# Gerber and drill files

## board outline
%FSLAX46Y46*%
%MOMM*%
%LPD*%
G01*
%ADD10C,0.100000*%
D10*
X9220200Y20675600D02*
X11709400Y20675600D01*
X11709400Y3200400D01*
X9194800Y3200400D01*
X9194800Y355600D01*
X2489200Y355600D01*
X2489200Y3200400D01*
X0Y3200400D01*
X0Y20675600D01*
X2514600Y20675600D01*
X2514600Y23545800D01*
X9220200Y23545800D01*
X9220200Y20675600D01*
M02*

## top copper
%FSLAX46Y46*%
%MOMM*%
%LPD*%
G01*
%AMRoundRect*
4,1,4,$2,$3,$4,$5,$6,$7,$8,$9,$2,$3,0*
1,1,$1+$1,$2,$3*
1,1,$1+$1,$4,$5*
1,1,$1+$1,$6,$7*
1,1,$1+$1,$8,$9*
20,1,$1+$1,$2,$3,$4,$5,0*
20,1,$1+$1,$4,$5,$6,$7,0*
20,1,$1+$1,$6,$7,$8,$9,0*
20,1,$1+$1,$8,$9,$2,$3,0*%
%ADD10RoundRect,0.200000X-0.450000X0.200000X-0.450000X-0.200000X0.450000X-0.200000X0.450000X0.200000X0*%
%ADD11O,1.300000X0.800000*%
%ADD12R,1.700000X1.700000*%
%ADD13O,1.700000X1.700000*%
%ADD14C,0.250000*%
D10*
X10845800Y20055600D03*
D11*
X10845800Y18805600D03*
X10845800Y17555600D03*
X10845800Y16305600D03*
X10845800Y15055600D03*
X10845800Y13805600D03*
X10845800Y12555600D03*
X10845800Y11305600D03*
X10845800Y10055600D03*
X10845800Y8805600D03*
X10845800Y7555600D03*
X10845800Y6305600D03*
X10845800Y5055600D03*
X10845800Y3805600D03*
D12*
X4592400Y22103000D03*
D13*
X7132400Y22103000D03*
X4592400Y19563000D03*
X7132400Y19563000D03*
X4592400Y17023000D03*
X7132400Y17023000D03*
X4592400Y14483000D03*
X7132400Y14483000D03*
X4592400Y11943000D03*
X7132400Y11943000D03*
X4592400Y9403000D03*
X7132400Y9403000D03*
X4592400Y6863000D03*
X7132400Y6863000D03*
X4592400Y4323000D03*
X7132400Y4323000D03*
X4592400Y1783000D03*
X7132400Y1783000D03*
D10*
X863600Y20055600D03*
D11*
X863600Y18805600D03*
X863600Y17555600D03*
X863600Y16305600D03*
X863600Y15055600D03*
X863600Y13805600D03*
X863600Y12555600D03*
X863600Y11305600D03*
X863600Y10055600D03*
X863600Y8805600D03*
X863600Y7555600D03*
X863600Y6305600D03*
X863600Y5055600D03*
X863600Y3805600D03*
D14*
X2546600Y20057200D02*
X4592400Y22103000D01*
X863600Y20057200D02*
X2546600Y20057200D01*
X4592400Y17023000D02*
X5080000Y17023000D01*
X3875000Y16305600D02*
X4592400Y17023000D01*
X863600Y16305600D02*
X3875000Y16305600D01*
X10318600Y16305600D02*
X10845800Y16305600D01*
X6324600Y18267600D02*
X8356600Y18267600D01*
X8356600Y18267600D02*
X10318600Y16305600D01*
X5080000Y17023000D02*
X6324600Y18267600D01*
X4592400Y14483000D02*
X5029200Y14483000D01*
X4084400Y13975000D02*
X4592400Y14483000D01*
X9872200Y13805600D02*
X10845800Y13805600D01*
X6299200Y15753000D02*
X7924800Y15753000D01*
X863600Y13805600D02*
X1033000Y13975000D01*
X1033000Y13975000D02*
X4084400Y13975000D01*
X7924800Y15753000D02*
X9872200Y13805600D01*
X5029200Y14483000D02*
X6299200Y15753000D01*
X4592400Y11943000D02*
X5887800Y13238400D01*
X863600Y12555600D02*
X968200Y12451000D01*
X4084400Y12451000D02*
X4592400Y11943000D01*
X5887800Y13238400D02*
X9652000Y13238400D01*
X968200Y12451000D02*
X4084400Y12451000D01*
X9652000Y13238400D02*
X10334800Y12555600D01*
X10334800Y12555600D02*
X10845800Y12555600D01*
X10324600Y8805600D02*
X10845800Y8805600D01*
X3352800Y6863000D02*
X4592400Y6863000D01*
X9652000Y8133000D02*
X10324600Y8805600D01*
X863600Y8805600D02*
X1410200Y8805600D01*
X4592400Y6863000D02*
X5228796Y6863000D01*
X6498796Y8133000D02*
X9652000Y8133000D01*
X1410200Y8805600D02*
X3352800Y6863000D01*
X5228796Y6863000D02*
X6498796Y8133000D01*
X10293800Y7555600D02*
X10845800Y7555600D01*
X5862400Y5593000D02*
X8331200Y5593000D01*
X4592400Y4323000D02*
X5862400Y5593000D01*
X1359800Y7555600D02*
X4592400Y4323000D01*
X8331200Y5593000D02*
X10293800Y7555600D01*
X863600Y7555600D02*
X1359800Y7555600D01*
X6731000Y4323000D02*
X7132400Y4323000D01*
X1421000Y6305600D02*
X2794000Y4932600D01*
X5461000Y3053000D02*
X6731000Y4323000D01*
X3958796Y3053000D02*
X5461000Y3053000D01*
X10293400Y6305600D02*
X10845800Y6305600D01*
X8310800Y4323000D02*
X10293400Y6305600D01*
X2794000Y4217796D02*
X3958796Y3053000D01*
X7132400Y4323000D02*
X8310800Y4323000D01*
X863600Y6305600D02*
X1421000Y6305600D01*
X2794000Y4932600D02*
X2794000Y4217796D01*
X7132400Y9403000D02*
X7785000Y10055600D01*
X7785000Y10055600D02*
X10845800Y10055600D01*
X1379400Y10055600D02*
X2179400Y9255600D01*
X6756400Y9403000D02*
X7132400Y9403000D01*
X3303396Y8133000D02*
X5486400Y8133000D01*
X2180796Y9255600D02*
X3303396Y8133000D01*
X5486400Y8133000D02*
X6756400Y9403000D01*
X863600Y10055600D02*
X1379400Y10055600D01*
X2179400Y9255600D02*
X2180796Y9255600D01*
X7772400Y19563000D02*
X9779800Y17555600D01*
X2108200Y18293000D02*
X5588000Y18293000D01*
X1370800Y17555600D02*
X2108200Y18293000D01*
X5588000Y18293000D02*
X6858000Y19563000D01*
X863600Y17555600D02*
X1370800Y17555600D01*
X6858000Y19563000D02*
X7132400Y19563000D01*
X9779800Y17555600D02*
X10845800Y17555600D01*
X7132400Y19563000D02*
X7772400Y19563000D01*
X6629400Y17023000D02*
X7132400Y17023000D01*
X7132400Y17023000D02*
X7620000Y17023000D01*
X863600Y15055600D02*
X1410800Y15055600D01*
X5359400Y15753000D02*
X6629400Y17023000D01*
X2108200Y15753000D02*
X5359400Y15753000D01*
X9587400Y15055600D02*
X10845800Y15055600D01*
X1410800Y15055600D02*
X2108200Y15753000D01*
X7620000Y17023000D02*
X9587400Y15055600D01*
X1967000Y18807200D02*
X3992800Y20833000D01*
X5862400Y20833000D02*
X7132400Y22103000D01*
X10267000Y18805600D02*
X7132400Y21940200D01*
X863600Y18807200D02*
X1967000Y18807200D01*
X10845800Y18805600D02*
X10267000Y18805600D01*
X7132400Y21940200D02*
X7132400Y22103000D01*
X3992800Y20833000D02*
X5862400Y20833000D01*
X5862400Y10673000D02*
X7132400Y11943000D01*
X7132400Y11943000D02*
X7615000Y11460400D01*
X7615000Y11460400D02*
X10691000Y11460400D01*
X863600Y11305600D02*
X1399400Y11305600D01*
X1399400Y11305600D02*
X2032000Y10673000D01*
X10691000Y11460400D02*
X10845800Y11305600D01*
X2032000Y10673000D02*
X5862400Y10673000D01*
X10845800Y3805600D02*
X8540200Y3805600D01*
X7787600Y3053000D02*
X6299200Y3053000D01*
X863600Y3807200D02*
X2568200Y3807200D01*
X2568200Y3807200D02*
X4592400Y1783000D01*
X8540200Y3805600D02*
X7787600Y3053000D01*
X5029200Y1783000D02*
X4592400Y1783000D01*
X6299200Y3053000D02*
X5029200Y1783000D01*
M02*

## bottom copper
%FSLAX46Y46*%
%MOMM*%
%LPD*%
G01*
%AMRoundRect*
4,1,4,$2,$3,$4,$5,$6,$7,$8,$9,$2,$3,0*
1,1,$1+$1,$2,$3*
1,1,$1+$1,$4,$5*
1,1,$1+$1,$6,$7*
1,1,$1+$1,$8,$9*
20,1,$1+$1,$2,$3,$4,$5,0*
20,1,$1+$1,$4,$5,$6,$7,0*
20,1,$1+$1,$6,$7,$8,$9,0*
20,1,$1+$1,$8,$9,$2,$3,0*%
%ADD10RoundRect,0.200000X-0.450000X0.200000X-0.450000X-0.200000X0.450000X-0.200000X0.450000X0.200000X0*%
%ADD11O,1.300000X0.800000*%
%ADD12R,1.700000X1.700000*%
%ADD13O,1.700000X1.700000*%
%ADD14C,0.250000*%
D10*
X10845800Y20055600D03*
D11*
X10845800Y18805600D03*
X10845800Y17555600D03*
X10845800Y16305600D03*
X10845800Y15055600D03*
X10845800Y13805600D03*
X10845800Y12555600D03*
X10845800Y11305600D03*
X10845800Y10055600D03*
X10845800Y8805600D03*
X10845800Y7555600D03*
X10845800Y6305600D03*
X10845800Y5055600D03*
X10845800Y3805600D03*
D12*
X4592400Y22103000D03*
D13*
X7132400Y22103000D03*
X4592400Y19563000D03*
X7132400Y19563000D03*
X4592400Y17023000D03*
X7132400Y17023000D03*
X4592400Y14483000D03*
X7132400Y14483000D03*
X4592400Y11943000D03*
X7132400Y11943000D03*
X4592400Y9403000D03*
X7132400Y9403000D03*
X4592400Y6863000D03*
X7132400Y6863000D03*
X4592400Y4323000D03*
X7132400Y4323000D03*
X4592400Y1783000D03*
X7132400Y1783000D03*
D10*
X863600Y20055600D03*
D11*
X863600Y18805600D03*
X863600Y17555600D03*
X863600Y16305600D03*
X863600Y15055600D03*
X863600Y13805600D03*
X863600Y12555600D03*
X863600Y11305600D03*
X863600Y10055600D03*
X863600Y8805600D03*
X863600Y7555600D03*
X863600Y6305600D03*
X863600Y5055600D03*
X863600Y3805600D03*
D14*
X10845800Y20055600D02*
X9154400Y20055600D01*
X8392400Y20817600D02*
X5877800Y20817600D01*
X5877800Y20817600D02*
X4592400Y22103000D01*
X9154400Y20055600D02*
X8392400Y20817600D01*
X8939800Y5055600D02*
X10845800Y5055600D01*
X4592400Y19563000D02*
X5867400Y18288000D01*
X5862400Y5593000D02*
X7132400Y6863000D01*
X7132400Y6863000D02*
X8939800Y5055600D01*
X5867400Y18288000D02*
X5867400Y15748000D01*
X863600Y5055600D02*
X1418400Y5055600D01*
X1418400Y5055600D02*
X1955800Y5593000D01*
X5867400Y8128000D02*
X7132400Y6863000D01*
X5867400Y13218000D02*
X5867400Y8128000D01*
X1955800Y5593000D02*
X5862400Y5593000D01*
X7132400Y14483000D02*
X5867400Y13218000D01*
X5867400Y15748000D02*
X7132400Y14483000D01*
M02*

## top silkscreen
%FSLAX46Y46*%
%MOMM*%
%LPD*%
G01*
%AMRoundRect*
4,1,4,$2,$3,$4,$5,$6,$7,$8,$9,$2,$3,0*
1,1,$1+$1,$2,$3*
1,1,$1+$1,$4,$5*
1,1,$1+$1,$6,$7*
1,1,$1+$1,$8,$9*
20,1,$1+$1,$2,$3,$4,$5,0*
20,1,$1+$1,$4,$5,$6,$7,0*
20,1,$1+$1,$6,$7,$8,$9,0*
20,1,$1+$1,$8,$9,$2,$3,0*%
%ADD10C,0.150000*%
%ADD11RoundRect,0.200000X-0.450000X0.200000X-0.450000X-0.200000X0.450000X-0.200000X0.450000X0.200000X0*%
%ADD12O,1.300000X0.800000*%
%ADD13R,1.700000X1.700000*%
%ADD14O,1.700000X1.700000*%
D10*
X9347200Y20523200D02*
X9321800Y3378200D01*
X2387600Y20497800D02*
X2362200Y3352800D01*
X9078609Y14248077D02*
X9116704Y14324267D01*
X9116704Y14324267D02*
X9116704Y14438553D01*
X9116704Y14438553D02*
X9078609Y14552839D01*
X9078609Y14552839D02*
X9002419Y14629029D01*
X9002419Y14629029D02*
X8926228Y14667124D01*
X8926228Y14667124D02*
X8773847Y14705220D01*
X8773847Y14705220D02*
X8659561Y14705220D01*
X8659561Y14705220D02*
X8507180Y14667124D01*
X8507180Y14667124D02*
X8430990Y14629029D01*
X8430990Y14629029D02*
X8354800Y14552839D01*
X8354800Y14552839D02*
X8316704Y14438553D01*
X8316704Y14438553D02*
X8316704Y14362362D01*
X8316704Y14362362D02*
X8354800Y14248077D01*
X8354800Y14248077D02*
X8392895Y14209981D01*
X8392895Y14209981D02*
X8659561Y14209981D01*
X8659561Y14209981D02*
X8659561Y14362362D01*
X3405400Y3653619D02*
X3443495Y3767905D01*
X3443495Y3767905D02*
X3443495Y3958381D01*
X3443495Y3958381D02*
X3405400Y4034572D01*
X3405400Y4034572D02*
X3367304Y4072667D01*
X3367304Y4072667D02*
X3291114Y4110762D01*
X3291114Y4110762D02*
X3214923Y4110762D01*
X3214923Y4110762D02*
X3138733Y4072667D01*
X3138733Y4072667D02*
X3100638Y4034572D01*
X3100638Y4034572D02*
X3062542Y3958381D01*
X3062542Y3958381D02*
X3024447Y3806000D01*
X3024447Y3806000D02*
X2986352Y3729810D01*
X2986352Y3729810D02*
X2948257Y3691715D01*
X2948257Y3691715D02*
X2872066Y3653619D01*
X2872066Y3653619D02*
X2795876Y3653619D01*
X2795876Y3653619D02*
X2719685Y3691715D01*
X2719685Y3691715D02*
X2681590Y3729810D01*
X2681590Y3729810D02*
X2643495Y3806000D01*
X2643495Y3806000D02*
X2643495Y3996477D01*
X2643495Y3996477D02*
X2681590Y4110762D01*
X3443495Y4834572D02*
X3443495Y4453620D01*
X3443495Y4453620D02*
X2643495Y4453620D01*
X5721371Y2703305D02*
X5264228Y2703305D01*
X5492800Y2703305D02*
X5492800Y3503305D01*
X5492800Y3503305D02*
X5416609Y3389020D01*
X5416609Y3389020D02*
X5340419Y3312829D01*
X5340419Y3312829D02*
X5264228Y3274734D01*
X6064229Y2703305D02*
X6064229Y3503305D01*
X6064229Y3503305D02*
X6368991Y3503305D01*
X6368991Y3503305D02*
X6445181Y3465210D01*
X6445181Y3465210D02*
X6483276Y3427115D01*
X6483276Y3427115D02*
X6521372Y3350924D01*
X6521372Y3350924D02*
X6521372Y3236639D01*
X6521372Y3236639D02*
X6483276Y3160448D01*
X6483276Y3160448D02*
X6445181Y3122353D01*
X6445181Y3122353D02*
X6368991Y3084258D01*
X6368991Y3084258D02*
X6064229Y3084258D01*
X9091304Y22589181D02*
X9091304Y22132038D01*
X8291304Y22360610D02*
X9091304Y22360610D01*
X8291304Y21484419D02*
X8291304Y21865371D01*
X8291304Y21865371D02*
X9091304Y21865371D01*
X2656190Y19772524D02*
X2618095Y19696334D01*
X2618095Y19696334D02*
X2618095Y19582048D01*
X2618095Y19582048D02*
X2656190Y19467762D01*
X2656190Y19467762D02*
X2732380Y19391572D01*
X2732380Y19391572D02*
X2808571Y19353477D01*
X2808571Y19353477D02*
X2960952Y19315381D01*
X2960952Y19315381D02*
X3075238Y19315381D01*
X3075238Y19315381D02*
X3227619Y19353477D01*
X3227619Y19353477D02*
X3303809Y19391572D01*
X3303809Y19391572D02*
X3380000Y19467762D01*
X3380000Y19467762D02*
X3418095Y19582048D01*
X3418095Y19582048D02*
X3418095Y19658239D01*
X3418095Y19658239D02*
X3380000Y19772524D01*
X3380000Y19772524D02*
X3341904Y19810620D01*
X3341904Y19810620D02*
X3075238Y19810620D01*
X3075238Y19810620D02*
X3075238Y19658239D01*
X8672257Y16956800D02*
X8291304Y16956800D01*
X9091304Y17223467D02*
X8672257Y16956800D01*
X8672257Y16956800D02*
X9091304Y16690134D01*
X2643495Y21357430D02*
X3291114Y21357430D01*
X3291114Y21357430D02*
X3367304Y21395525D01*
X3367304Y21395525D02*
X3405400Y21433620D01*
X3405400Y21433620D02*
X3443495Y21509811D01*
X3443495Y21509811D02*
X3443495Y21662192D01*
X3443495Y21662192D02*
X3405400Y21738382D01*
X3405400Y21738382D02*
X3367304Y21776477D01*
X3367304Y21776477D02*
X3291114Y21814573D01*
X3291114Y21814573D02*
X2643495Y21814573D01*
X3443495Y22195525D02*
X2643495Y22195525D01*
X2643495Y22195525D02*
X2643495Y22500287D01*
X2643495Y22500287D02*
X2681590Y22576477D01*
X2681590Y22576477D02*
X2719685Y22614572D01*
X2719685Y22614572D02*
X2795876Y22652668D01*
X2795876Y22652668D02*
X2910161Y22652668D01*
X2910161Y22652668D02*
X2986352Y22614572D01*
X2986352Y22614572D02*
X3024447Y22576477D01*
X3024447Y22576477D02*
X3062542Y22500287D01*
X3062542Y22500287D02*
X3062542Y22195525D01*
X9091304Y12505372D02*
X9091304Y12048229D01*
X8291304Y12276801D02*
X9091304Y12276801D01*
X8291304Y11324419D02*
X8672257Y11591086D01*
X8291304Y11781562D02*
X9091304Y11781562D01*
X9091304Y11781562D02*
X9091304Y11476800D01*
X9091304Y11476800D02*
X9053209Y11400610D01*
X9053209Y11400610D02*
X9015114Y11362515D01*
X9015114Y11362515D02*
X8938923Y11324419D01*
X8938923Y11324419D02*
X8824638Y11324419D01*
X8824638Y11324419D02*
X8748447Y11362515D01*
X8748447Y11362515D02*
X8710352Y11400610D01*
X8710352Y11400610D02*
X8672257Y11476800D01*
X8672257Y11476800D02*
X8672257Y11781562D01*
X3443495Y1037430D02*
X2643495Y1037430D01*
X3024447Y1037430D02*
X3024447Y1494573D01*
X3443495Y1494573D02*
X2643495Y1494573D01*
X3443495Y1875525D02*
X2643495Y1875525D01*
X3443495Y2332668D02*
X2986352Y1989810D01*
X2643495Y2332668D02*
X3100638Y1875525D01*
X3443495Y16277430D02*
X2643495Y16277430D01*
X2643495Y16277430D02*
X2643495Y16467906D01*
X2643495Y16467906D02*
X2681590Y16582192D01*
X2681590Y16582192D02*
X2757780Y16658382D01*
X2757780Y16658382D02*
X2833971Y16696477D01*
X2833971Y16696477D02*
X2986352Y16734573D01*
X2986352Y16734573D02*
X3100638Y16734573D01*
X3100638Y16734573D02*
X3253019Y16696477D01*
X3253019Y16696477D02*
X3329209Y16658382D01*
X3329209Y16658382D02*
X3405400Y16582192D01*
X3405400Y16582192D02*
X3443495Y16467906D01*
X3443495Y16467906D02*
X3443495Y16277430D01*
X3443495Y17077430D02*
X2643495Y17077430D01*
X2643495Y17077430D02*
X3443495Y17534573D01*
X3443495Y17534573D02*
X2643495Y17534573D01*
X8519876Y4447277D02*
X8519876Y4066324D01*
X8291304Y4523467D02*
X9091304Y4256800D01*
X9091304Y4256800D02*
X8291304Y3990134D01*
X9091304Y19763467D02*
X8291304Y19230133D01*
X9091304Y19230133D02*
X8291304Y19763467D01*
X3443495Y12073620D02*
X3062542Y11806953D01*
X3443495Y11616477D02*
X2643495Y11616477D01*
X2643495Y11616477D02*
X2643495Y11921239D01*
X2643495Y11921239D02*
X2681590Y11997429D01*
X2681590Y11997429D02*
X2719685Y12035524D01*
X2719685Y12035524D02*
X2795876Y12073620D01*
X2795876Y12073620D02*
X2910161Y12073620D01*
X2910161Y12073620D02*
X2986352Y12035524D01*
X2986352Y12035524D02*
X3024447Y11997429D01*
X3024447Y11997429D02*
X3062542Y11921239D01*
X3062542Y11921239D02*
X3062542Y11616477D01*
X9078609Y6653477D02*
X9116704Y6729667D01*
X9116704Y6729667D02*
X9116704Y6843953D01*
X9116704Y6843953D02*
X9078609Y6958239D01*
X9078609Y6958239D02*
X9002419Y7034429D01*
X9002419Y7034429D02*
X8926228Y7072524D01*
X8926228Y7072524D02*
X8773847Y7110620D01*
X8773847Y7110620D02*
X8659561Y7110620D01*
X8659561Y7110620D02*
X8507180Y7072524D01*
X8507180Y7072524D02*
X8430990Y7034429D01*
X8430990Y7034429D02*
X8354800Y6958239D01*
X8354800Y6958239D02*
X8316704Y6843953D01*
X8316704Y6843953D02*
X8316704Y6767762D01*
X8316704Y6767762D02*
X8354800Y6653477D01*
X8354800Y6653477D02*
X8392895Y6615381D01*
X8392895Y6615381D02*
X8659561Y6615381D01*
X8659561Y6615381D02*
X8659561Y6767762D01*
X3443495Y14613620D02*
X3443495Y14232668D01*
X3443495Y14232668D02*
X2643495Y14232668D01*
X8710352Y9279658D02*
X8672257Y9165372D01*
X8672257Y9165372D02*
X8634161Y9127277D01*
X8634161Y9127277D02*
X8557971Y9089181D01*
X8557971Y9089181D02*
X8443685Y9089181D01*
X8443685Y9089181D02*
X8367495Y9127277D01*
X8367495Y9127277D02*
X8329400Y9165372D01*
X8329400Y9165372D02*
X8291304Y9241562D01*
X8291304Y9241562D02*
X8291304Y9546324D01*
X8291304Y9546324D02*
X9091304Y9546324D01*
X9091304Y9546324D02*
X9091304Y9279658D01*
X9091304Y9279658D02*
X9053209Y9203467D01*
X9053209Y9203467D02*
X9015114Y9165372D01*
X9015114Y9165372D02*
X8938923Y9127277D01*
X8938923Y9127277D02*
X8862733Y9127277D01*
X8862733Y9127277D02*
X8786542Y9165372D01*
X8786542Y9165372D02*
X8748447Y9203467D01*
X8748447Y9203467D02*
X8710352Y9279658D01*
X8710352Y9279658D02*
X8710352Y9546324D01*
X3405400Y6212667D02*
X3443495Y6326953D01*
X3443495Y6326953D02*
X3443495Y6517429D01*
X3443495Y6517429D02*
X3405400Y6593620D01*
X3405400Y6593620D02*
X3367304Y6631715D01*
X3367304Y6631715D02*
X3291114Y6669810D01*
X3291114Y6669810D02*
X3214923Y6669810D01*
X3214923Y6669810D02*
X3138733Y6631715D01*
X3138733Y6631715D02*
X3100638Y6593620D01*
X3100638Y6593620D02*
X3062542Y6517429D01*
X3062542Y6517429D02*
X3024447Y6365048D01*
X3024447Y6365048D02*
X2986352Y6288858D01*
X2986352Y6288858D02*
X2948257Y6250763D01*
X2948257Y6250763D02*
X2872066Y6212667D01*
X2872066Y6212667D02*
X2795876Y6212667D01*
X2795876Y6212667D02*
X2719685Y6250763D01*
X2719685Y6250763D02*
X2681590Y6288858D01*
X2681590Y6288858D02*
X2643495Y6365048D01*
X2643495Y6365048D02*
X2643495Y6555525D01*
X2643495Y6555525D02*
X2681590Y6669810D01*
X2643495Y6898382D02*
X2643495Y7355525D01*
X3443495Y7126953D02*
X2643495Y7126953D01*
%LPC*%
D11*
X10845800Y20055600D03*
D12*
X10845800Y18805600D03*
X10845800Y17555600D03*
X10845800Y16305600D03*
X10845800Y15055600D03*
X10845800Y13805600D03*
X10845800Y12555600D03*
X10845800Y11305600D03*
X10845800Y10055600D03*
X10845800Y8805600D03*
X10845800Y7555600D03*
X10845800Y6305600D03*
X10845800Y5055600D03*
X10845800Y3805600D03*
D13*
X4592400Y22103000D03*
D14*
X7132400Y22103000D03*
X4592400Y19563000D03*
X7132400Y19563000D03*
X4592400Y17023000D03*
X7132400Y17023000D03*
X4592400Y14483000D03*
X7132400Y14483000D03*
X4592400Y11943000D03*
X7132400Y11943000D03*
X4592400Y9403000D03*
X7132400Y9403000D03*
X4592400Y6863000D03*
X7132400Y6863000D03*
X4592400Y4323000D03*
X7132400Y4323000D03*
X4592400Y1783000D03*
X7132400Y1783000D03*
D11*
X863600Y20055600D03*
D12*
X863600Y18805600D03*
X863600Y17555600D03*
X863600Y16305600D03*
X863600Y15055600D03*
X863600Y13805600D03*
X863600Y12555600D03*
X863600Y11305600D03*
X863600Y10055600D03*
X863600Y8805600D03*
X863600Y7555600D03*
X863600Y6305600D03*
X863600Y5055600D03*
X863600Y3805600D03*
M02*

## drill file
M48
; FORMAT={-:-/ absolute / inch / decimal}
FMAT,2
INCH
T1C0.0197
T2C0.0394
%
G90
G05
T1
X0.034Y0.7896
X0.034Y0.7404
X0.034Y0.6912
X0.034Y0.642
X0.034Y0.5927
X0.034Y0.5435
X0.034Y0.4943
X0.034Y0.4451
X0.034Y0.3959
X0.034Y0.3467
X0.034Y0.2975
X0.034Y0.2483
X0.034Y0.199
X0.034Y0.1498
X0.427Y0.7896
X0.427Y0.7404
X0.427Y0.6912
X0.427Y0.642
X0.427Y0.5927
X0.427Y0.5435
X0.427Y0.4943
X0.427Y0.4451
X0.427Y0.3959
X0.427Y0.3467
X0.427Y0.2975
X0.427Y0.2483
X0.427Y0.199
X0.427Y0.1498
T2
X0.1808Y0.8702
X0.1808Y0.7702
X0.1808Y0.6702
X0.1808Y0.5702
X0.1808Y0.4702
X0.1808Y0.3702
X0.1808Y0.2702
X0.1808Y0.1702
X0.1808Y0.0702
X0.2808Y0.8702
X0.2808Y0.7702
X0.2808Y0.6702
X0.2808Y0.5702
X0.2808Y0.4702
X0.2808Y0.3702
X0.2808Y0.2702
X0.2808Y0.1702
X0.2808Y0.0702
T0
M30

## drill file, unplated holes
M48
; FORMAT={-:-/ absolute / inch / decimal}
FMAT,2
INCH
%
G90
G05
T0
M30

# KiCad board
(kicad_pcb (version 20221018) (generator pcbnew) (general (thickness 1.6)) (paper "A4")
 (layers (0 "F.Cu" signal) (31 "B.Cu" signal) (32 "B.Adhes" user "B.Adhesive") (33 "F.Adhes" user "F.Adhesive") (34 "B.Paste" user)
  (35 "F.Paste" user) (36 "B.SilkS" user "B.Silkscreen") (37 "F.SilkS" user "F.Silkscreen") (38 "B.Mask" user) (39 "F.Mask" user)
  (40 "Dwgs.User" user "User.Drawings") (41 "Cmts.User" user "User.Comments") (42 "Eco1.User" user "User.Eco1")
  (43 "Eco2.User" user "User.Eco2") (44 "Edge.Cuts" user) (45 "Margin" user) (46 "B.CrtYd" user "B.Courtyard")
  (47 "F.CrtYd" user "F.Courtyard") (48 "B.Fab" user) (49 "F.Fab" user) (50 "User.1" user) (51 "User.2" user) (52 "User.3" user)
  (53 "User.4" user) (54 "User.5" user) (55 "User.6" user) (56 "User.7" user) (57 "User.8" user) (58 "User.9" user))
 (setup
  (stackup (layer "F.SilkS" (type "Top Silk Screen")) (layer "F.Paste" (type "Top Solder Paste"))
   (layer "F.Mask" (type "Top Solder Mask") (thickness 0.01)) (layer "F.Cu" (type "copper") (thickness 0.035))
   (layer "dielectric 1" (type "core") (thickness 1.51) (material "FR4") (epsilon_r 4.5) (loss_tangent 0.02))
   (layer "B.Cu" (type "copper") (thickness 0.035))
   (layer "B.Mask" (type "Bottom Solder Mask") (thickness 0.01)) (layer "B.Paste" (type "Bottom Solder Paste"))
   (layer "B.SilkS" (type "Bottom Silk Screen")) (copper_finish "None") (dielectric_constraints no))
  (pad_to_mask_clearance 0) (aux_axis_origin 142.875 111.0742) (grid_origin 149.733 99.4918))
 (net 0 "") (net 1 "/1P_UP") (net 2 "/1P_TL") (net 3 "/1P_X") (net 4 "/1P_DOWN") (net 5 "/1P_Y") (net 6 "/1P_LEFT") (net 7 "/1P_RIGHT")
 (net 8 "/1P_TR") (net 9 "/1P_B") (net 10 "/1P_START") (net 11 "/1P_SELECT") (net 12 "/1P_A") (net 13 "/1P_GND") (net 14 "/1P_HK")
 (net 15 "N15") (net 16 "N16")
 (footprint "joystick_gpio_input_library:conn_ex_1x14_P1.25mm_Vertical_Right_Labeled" (layer "B.Cu") (at 153.7208 91.0186 -90)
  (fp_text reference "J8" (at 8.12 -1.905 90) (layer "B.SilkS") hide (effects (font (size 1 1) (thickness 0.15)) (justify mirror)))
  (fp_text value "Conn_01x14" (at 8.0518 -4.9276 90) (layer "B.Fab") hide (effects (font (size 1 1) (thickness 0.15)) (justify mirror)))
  (pad "1" thru_hole roundrect (at 0 0 270) (size 0.8 1.3) (drill 0.5) (layers "*.Cu" "*.Mask") (roundrect_rratio 0.25) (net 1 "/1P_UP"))
  (pad "2" thru_hole oval (at 1.25 0 270) (size 0.8 1.3) (drill 0.5) (layers "*.Cu" "*.Mask") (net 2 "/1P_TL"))
  (pad "3" thru_hole oval (at 2.5 0 270) (size 0.8 1.3) (drill 0.5) (layers "*.Cu" "*.Mask") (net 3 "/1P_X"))
  (pad "4" thru_hole oval (at 3.75 0 270) (size 0.8 1.3) (drill 0.5) (layers "*.Cu" "*.Mask") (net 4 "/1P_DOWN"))
  (pad "5" thru_hole oval (at 5 0 270) (size 0.8 1.3) (drill 0.5) (layers "*.Cu" "*.Mask") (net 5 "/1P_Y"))
  (pad "6" thru_hole oval (at 6.25 0 270) (size 0.8 1.3) (drill 0.5) (layers "*.Cu" "*.Mask") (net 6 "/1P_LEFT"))
  (pad "7" thru_hole oval (at 7.5 0 270) (size 0.8 1.3) (drill 0.5) (layers "*.Cu" "*.Mask") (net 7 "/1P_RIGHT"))
  (pad "8" thru_hole oval (at 8.75 0 270) (size 0.8 1.3) (drill 0.5) (layers "*.Cu" "*.Mask") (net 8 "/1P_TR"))
  (pad "9" thru_hole oval (at 10 0 270) (size 0.8 1.3) (drill 0.5) (layers "*.Cu" "*.Mask") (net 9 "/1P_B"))
  (pad "10" thru_hole oval (at 11.25 0 270) (size 0.8 1.3) (drill 0.5) (layers "*.Cu" "*.Mask") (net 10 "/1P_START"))
  (pad "11" thru_hole oval (at 12.5 0 270) (size 0.8 1.3) (drill 0.5) (layers "*.Cu" "*.Mask") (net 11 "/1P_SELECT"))
  (pad "12" thru_hole oval (at 13.75 0 270) (size 0.8 1.3) (drill 0.5) (layers "*.Cu" "*.Mask") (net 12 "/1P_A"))
  (pad "13" thru_hole oval (at 15 0 270) (size 0.8 1.3) (drill 0.5) (layers "*.Cu" "*.Mask") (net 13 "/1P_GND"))
  (pad "14" thru_hole oval (at 16.25 0 270) (size 0.8 1.3) (drill 0.5) (layers "*.Cu" "*.Mask") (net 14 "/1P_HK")))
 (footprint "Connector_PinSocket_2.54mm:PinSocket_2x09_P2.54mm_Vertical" (layer "B.Cu") (at 147.4674 88.9712 180)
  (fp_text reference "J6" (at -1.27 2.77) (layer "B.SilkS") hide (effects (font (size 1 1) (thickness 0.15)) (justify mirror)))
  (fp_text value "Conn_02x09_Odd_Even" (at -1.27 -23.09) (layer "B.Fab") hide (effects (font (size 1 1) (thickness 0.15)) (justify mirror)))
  (pad "1" thru_hole rect (at 0 0 180) (size 1.7 1.7) (drill 1) (layers "*.Cu" "*.Mask") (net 1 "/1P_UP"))
  (pad "2" thru_hole oval (at -2.54 0 180) (size 1.7 1.7) (drill 1) (layers "*.Cu" "*.Mask") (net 2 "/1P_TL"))
  (pad "3" thru_hole oval (at 0 -2.54 180) (size 1.7 1.7) (drill 1) (layers "*.Cu" "*.Mask") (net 13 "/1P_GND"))
  (pad "4" thru_hole oval (at -2.54 -2.54 180) (size 1.7 1.7) (drill 1) (layers "*.Cu" "*.Mask") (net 3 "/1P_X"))
  (pad "5" thru_hole oval (at 0 -5.08 180) (size 1.7 1.7) (drill 1) (layers "*.Cu" "*.Mask") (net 4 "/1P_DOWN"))
  (pad "6" thru_hole oval (at -2.54 -5.08 180) (size 1.7 1.7) (drill 1) (layers "*.Cu" "*.Mask") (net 5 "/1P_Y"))
  (pad "7" thru_hole oval (at 0 -7.62 180) (size 1.7 1.7) (drill 1) (layers "*.Cu" "*.Mask") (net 6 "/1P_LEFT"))
  (pad "8" thru_hole oval (at -2.54 -7.62 180) (size 1.7 1.7) (drill 1) (layers "*.Cu" "*.Mask") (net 13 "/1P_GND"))
  (pad "9" thru_hole oval (at 0 -10.16 180) (size 1.7 1.7) (drill 1) (layers "*.Cu" "*.Mask") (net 7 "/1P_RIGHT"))
  (pad "10" thru_hole oval (at -2.54 -10.16 180) (size 1.7 1.7) (drill 1) (layers "*.Cu" "*.Mask") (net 8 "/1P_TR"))
  (pad "11" thru_hole oval (at 0 -12.7 180) (size 1.7 1.7) (drill 1) (layers "*.Cu" "*.Mask") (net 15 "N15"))
  (pad "12" thru_hole oval (at -2.54 -12.7 180) (size 1.7 1.7) (drill 1) (layers "*.Cu" "*.Mask") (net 9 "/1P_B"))
  (pad "13" thru_hole oval (at 0 -15.24 180) (size 1.7 1.7) (drill 1) (layers "*.Cu" "*.Mask") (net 10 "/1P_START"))
  (pad "14" thru_hole oval (at -2.54 -15.24 180) (size 1.7 1.7) (drill 1) (layers "*.Cu" "*.Mask") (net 13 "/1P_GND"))
  (pad "15" thru_hole oval (at 0 -17.78 180) (size 1.7 1.7) (drill 1) (layers "*.Cu" "*.Mask") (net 11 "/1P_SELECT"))
  (pad "16" thru_hole oval (at -2.54 -17.78 180) (size 1.7 1.7) (drill 1) (layers "*.Cu" "*.Mask") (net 12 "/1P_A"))
  (pad "17" thru_hole oval (at 0 -20.32 180) (size 1.7 1.7) (drill 1) (layers "*.Cu" "*.Mask") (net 14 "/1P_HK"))
  (pad "18" thru_hole oval (at -2.54 -20.32 180) (size 1.7 1.7) (drill 1) (layers "*.Cu" "*.Mask") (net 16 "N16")))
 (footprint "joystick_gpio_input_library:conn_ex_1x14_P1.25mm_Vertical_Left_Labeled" (layer "B.Cu") (at 143.7386 91.0186 -90)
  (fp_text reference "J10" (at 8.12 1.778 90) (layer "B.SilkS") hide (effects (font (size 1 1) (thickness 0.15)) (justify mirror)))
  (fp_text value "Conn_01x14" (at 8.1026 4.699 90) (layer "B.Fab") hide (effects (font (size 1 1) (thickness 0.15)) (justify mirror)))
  (pad "1" thru_hole roundrect (at 0 0 270) (size 0.8 1.3) (drill 0.5) (layers "*.Cu" "*.Mask") (roundrect_rratio 0.25) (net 1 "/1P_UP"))
  (pad "2" thru_hole oval (at 1.25 0 270) (size 0.8 1.3) (drill 0.5) (layers "*.Cu" "*.Mask") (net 2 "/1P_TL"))
  (pad "3" thru_hole oval (at 2.5 0 270) (size 0.8 1.3) (drill 0.5) (layers "*.Cu" "*.Mask") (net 3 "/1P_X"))
  (pad "4" thru_hole oval (at 3.75 0 270) (size 0.8 1.3) (drill 0.5) (layers "*.Cu" "*.Mask") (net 4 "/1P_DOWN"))
  (pad "5" thru_hole oval (at 5 0 270) (size 0.8 1.3) (drill 0.5) (layers "*.Cu" "*.Mask") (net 5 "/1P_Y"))
  (pad "6" thru_hole oval (at 6.25 0 270) (size 0.8 1.3) (drill 0.5) (layers "*.Cu" "*.Mask") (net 6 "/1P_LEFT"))
  (pad "7" thru_hole oval (at 7.5 0 270) (size 0.8 1.3) (drill 0.5) (layers "*.Cu" "*.Mask") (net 7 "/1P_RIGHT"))
  (pad "8" thru_hole oval (at 8.75 0 270) (size 0.8 1.3) (drill 0.5) (layers "*.Cu" "*.Mask") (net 8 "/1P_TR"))
  (pad "9" thru_hole oval (at 10 0 270) (size 0.8 1.3) (drill 0.5) (layers "*.Cu" "*.Mask") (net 9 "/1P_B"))
  (pad "10" thru_hole oval (at 11.25 0 270) (size 0.8 1.3) (drill 0.5) (layers "*.Cu" "*.Mask") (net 10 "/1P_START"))
  (pad "11" thru_hole oval (at 12.5 0 270) (size 0.8 1.3) (drill 0.5) (layers "*.Cu" "*.Mask") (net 11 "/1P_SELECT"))
  (pad "12" thru_hole oval (at 13.75 0 270) (size 0.8 1.3) (drill 0.5) (layers "*.Cu" "*.Mask") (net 12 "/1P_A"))
  (pad "13" thru_hole oval (at 15 0 270) (size 0.8 1.3) (drill 0.5) (layers "*.Cu" "*.Mask") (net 13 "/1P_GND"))
  (pad "14" thru_hole oval (at 16.25 0 270) (size 0.8 1.3) (drill 0.5) (layers "*.Cu" "*.Mask") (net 14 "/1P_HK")))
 (gr_line (start 152.2222 90.551) (end 152.1968 107.696) (stroke (width 0.15) (type default)) (layer "F.SilkS"))
 (gr_line (start 145.2626 90.5764) (end 145.2372 107.7214) (stroke (width 0.15) (type default)) (layer "F.SilkS"))
 (gr_poly
  (pts (xy 152.0952 87.5284) (xy 145.3896 87.5284) (xy 145.3896 90.3986) (xy 142.875 90.3986) (xy 142.875 107.8738) (xy 145.3642 107.8738)
   (xy 145.3642 110.7186) (xy 152.0698 110.7186) (xy 152.0698 107.8738) (xy 154.5844 107.8738) (xy 154.5844 90.3986) (xy 152.0952 90.3986))
  (stroke (width 0.1) (type solid)) (fill none) (layer "Edge.Cuts"))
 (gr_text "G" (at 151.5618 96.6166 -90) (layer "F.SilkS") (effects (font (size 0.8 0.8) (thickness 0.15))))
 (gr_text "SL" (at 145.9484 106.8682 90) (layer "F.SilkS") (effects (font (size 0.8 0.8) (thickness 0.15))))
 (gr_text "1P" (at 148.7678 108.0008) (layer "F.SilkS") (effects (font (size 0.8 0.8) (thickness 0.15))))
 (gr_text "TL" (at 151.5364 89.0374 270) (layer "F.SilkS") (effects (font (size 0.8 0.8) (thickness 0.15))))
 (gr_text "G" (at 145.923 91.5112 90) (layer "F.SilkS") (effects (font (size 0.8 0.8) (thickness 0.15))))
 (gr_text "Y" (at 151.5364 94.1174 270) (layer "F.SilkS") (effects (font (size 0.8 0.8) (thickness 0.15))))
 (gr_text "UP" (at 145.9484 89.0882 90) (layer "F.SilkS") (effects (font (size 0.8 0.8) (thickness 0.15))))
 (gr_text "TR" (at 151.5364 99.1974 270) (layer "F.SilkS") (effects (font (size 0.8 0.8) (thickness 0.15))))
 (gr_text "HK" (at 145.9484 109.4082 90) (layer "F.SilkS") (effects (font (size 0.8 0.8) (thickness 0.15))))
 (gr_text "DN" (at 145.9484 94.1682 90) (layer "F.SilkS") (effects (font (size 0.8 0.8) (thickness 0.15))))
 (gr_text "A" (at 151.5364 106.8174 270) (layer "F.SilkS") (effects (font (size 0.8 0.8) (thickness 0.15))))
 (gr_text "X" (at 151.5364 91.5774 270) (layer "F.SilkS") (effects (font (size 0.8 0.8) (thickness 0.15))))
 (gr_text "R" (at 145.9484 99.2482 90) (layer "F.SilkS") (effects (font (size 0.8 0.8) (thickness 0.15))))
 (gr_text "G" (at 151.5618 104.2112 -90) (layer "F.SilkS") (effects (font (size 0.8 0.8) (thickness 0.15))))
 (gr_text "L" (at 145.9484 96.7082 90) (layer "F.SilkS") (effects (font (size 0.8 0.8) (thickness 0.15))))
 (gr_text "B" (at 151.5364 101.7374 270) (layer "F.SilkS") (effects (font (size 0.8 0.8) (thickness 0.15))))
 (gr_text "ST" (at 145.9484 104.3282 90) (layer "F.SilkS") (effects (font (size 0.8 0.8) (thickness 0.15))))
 (segment (start 145.4216 91.017) (end 147.4674 88.9712) (width 0.25) (layer "F.Cu") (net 1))
 (segment (start 143.7386 91.017) (end 145.4216 91.017) (width 0.25) (layer "F.Cu") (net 1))
 (segment (start 153.7208 91.0186) (end 152.0294 91.0186) (width 0.25) (layer "B.Cu") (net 1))
 (segment (start 151.2674 90.2566) (end 148.7528 90.2566) (width 0.25) (layer "B.Cu") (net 1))
 (segment (start 148.7528 90.2566) (end 147.4674 88.9712) (width 0.25) (layer "B.Cu") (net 1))
 (segment (start 152.0294 91.0186) (end 151.2674 90.2566) (width 0.25) (layer "B.Cu") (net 1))
 (segment (start 147.4674 94.0512) (end 147.955 94.0512) (width 0.25) (layer "F.Cu") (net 4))
 (segment (start 146.75 94.7686) (end 147.4674 94.0512) (width 0.25) (layer "F.Cu") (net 4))
 (segment (start 143.7386 94.7686) (end 146.75 94.7686) (width 0.25) (layer "F.Cu") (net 4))
 (segment (start 153.1936 94.7686) (end 153.7208 94.7686) (width 0.25) (layer "F.Cu") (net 4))
 (segment (start 149.1996 92.8066) (end 151.2316 92.8066) (width 0.25) (layer "F.Cu") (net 4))
 (segment (start 151.2316 92.8066) (end 153.1936 94.7686) (width 0.25) (layer "F.Cu") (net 4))
 (segment (start 147.955 94.0512) (end 149.1996 92.8066) (width 0.25) (layer "F.Cu") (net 4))
 (segment (start 147.4674 96.5912) (end 147.9042 96.5912) (width 0.25) (layer "F.Cu") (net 6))
 (segment (start 146.9594 97.0992) (end 147.4674 96.5912) (width 0.25) (layer "F.Cu") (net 6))
 (segment (start 152.7472 97.2686) (end 153.7208 97.2686) (width 0.25) (layer "F.Cu") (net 6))
 (segment (start 149.1742 95.3212) (end 150.7998 95.3212) (width 0.25) (layer "F.Cu") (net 6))
 (segment (start 143.7386 97.2686) (end 143.908 97.0992) (width 0.25) (layer "F.Cu") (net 6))
 (segment (start 143.908 97.0992) (end 146.9594 97.0992) (width 0.25) (layer "F.Cu") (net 6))
 (segment (start 150.7998 95.3212) (end 152.7472 97.2686) (width 0.25) (layer "F.Cu") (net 6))
 (segment (start 147.9042 96.5912) (end 149.1742 95.3212) (width 0.25) (layer "F.Cu") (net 6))
 (segment (start 147.4674 99.1312) (end 148.7628 97.8358) (width 0.25) (layer "F.Cu") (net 7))
 (segment (start 143.7386 98.5186) (end 143.8432 98.6232) (width 0.25) (layer "F.Cu") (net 7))
 (segment (start 146.9594 98.6232) (end 147.4674 99.1312) (width 0.25) (layer "F.Cu") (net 7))
 (segment (start 148.7628 97.8358) (end 152.527 97.8358) (width 0.25) (layer "F.Cu") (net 7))
 (segment (start 143.8432 98.6232) (end 146.9594 98.6232) (width 0.25) (layer "F.Cu") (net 7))
 (segment (start 152.527 97.8358) (end 153.2098 98.5186) (width 0.25) (layer "F.Cu") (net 7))
 (segment (start 153.2098 98.5186) (end 153.7208 98.5186) (width 0.25) (layer "F.Cu") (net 7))
 (segment (start 153.1996 102.2686) (end 153.7208 102.2686) (width 0.25) (layer "F.Cu") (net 10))
 (segment (start 146.2278 104.2112) (end 147.4674 104.2112) (width 0.25) (layer "F.Cu") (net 10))
 (segment (start 152.527 102.9412) (end 153.1996 102.2686) (width 0.25) (layer "F.Cu") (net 10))
 (segment (start 143.7386 102.2686) (end 144.2852 102.2686) (width 0.25) (layer "F.Cu") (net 10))
 (segment (start 147.4674 104.2112) (end 148.103796 104.2112) (width 0.25) (layer "F.Cu") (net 10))
 (segment (start 149.373796 102.9412) (end 152.527 102.9412) (width 0.25) (layer "F.Cu") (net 10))
 (segment (start 144.2852 102.2686) (end 146.2278 104.2112) (width 0.25) (layer "F.Cu") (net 10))
 (segment (start 148.103796 104.2112) (end 149.373796 102.9412) (width 0.25) (layer "F.Cu") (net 10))
 (segment (start 153.1688 103.5186) (end 153.7208 103.5186) (width 0.25) (layer "F.Cu") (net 11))
 (segment (start 148.7374 105.4812) (end 151.2062 105.4812) (width 0.25) (layer "F.Cu") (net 11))
 (segment (start 147.4674 106.7512) (end 148.7374 105.4812) (width 0.25) (layer "F.Cu") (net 11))
 (segment (start 144.2348 103.5186) (end 147.4674 106.7512) (width 0.25) (layer "F.Cu") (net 11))
 (segment (start 151.2062 105.4812) (end 153.1688 103.5186) (width 0.25) (layer "F.Cu") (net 11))
 (segment (start 143.7386 103.5186) (end 144.2348 103.5186) (width 0.25) (layer "F.Cu") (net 11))
 (segment (start 149.606 106.7512) (end 150.0074 106.7512) (width 0.25) (layer "F.Cu") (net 12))
 (segment (start 144.296 104.7686) (end 145.669 106.1416) (width 0.25) (layer "F.Cu") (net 12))
 (segment (start 148.336 108.0212) (end 149.606 106.7512) (width 0.25) (layer "F.Cu") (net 12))
 (segment (start 146.833796 108.0212) (end 148.336 108.0212) (width 0.25) (layer "F.Cu") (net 12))
 (segment (start 153.1684 104.7686) (end 153.7208 104.7686) (width 0.25) (layer "F.Cu") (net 12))
 (segment (start 151.1858 106.7512) (end 153.1684 104.7686) (width 0.25) (layer "F.Cu") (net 12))
 (segment (start 145.669 106.856404) (end 146.833796 108.0212) (width 0.25) (layer "F.Cu") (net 12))
 (segment (start 150.0074 106.7512) (end 151.1858 106.7512) (width 0.25) (layer "F.Cu") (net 12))
 (segment (start 143.7386 104.7686) (end 144.296 104.7686) (width 0.25) (layer "F.Cu") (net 12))
 (segment (start 145.669 106.1416) (end 145.669 106.856404) (width 0.25) (layer "F.Cu") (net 12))
 (segment (start 150.0074 101.6712) (end 150.66 101.0186) (width 0.25) (layer "F.Cu") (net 9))
 (segment (start 150.66 101.0186) (end 153.7208 101.0186) (width 0.25) (layer "F.Cu") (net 9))
 (segment (start 144.2544 101.0186) (end 145.0544 101.8186) (width 0.25) (layer "F.Cu") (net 9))
 (segment (start 149.6314 101.6712) (end 150.0074 101.6712) (width 0.25) (layer "F.Cu") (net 9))
 (segment (start 146.178396 102.9412) (end 148.3614 102.9412) (width 0.25) (layer "F.Cu") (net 9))
 (segment (start 145.055796 101.8186) (end 146.178396 102.9412) (width 0.25) (layer "F.Cu") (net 9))
 (segment (start 148.3614 102.9412) (end 149.6314 101.6712) (width 0.25) (layer "F.Cu") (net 9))
 (segment (start 143.7386 101.0186) (end 144.2544 101.0186) (width 0.25) (layer "F.Cu") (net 9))
 (segment (start 145.0544 101.8186) (end 145.055796 101.8186) (width 0.25) (layer "F.Cu") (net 9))
 (segment (start 150.6474 91.5112) (end 152.6548 93.5186) (width 0.25) (layer "F.Cu") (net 3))
 (segment (start 144.9832 92.7812) (end 148.463 92.7812) (width 0.25) (layer "F.Cu") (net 3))
 (segment (start 144.2458 93.5186) (end 144.9832 92.7812) (width 0.25) (layer "F.Cu") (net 3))
 (segment (start 148.463 92.7812) (end 149.733 91.5112) (width 0.25) (layer "F.Cu") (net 3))
 (segment (start 143.7386 93.5186) (end 144.2458 93.5186) (width 0.25) (layer "F.Cu") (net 3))
 (segment (start 149.733 91.5112) (end 150.0074 91.5112) (width 0.25) (layer "F.Cu") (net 3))
 (segment (start 152.6548 93.5186) (end 153.7208 93.5186) (width 0.25) (layer "F.Cu") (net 3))
 (segment (start 150.0074 91.5112) (end 150.6474 91.5112) (width 0.25) (layer "F.Cu") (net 3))
 (segment (start 149.5044 94.0512) (end 150.0074 94.0512) (width 0.25) (layer "F.Cu") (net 5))
 (segment (start 150.0074 94.0512) (end 150.495 94.0512) (width 0.25) (layer "F.Cu") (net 5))
 (segment (start 143.7386 96.0186) (end 144.2858 96.0186) (width 0.25) (layer "F.Cu") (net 5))
 (segment (start 148.2344 95.3212) (end 149.5044 94.0512) (width 0.25) (layer "F.Cu") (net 5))
 (segment (start 144.9832 95.3212) (end 148.2344 95.3212) (width 0.25) (layer "F.Cu") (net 5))
 (segment (start 152.4624 96.0186) (end 153.7208 96.0186) (width 0.25) (layer "F.Cu") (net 5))
 (segment (start 144.2858 96.0186) (end 144.9832 95.3212) (width 0.25) (layer "F.Cu") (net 5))
 (segment (start 150.495 94.0512) (end 152.4624 96.0186) (width 0.25) (layer "F.Cu") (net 5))
 (segment (start 144.842 92.267) (end 146.8678 90.2412) (width 0.25) (layer "F.Cu") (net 2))
 (segment (start 148.7374 90.2412) (end 150.0074 88.9712) (width 0.25) (layer "F.Cu") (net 2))
 (segment (start 153.142 92.2686) (end 150.0074 89.134) (width 0.25) (layer "F.Cu") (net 2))
 (segment (start 143.7386 92.267) (end 144.842 92.267) (width 0.25) (layer "F.Cu") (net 2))
 (segment (start 153.7208 92.2686) (end 153.142 92.2686) (width 0.25) (layer "F.Cu") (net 2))
 (segment (start 150.0074 89.134) (end 150.0074 88.9712) (width 0.25) (layer "F.Cu") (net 2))
 (segment (start 146.8678 90.2412) (end 148.7374 90.2412) (width 0.25) (layer "F.Cu") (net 2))
 (segment (start 148.7374 100.4012) (end 150.0074 99.1312) (width 0.25) (layer "F.Cu") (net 8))
 (segment (start 150.0074 99.1312) (end 150.49 99.6138) (width 0.25) (layer "F.Cu") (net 8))
 (segment (start 150.49 99.6138) (end 153.566 99.6138) (width 0.25) (layer "F.Cu") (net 8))
 (segment (start 143.7386 99.7686) (end 144.2744 99.7686) (width 0.25) (layer "F.Cu") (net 8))
 (segment (start 144.2744 99.7686) (end 144.907 100.4012) (width 0.25) (layer "F.Cu") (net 8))
 (segment (start 153.566 99.6138) (end 153.7208 99.7686) (width 0.25) (layer "F.Cu") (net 8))
 (segment (start 144.907 100.4012) (end 148.7374 100.4012) (width 0.25) (layer "F.Cu") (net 8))
 (segment (start 153.7208 107.2686) (end 151.4152 107.2686) (width 0.25) (layer "F.Cu") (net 14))
 (segment (start 150.6626 108.0212) (end 149.1742 108.0212) (width 0.25) (layer "F.Cu") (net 14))
 (segment (start 143.7386 107.267) (end 145.4432 107.267) (width 0.25) (layer "F.Cu") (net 14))
 (segment (start 145.4432 107.267) (end 147.4674 109.2912) (width 0.25) (layer "F.Cu") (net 14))
 (segment (start 151.4152 107.2686) (end 150.6626 108.0212) (width 0.25) (layer "F.Cu") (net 14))
 (segment (start 147.9042 109.2912) (end 147.4674 109.2912) (width 0.25) (layer "F.Cu") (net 14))
 (segment (start 149.1742 108.0212) (end 147.9042 109.2912) (width 0.25) (layer "F.Cu") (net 14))
 (segment (start 151.8148 106.0186) (end 153.7208 106.0186) (width 0.25) (layer "B.Cu") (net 13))
 (segment (start 147.4674 91.5112) (end 148.7424 92.7862) (width 0.25) (layer "B.Cu") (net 13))
 (segment (start 148.7374 105.4812) (end 150.0074 104.2112) (width 0.25) (layer "B.Cu") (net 13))
 (segment (start 150.0074 104.2112) (end 151.8148 106.0186) (width 0.25) (layer "B.Cu") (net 13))
 (segment (start 148.7424 92.7862) (end 148.7424 95.3262) (width 0.25) (layer "B.Cu") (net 13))
 (segment (start 143.7386 106.0186) (end 144.2934 106.0186) (width 0.25) (layer "B.Cu") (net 13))
 (segment (start 144.2934 106.0186) (end 144.8308 105.4812) (width 0.25) (layer "B.Cu") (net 13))
 (segment (start 148.7424 102.9462) (end 150.0074 104.2112) (width 0.25) (layer "B.Cu") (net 13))
 (segment (start 148.7424 97.8562) (end 148.7424 102.9462) (width 0.25) (layer "B.Cu") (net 13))
 (segment (start 144.8308 105.4812) (end 148.7374 105.4812) (width 0.25) (layer "B.Cu") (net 13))
 (segment (start 150.0074 96.5912) (end 148.7424 97.8562) (width 0.25) (layer "B.Cu") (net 13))
 (segment (start 148.7424 95.3262) (end 150.0074 96.5912) (width 0.25) (layer "B.Cu") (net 13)))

